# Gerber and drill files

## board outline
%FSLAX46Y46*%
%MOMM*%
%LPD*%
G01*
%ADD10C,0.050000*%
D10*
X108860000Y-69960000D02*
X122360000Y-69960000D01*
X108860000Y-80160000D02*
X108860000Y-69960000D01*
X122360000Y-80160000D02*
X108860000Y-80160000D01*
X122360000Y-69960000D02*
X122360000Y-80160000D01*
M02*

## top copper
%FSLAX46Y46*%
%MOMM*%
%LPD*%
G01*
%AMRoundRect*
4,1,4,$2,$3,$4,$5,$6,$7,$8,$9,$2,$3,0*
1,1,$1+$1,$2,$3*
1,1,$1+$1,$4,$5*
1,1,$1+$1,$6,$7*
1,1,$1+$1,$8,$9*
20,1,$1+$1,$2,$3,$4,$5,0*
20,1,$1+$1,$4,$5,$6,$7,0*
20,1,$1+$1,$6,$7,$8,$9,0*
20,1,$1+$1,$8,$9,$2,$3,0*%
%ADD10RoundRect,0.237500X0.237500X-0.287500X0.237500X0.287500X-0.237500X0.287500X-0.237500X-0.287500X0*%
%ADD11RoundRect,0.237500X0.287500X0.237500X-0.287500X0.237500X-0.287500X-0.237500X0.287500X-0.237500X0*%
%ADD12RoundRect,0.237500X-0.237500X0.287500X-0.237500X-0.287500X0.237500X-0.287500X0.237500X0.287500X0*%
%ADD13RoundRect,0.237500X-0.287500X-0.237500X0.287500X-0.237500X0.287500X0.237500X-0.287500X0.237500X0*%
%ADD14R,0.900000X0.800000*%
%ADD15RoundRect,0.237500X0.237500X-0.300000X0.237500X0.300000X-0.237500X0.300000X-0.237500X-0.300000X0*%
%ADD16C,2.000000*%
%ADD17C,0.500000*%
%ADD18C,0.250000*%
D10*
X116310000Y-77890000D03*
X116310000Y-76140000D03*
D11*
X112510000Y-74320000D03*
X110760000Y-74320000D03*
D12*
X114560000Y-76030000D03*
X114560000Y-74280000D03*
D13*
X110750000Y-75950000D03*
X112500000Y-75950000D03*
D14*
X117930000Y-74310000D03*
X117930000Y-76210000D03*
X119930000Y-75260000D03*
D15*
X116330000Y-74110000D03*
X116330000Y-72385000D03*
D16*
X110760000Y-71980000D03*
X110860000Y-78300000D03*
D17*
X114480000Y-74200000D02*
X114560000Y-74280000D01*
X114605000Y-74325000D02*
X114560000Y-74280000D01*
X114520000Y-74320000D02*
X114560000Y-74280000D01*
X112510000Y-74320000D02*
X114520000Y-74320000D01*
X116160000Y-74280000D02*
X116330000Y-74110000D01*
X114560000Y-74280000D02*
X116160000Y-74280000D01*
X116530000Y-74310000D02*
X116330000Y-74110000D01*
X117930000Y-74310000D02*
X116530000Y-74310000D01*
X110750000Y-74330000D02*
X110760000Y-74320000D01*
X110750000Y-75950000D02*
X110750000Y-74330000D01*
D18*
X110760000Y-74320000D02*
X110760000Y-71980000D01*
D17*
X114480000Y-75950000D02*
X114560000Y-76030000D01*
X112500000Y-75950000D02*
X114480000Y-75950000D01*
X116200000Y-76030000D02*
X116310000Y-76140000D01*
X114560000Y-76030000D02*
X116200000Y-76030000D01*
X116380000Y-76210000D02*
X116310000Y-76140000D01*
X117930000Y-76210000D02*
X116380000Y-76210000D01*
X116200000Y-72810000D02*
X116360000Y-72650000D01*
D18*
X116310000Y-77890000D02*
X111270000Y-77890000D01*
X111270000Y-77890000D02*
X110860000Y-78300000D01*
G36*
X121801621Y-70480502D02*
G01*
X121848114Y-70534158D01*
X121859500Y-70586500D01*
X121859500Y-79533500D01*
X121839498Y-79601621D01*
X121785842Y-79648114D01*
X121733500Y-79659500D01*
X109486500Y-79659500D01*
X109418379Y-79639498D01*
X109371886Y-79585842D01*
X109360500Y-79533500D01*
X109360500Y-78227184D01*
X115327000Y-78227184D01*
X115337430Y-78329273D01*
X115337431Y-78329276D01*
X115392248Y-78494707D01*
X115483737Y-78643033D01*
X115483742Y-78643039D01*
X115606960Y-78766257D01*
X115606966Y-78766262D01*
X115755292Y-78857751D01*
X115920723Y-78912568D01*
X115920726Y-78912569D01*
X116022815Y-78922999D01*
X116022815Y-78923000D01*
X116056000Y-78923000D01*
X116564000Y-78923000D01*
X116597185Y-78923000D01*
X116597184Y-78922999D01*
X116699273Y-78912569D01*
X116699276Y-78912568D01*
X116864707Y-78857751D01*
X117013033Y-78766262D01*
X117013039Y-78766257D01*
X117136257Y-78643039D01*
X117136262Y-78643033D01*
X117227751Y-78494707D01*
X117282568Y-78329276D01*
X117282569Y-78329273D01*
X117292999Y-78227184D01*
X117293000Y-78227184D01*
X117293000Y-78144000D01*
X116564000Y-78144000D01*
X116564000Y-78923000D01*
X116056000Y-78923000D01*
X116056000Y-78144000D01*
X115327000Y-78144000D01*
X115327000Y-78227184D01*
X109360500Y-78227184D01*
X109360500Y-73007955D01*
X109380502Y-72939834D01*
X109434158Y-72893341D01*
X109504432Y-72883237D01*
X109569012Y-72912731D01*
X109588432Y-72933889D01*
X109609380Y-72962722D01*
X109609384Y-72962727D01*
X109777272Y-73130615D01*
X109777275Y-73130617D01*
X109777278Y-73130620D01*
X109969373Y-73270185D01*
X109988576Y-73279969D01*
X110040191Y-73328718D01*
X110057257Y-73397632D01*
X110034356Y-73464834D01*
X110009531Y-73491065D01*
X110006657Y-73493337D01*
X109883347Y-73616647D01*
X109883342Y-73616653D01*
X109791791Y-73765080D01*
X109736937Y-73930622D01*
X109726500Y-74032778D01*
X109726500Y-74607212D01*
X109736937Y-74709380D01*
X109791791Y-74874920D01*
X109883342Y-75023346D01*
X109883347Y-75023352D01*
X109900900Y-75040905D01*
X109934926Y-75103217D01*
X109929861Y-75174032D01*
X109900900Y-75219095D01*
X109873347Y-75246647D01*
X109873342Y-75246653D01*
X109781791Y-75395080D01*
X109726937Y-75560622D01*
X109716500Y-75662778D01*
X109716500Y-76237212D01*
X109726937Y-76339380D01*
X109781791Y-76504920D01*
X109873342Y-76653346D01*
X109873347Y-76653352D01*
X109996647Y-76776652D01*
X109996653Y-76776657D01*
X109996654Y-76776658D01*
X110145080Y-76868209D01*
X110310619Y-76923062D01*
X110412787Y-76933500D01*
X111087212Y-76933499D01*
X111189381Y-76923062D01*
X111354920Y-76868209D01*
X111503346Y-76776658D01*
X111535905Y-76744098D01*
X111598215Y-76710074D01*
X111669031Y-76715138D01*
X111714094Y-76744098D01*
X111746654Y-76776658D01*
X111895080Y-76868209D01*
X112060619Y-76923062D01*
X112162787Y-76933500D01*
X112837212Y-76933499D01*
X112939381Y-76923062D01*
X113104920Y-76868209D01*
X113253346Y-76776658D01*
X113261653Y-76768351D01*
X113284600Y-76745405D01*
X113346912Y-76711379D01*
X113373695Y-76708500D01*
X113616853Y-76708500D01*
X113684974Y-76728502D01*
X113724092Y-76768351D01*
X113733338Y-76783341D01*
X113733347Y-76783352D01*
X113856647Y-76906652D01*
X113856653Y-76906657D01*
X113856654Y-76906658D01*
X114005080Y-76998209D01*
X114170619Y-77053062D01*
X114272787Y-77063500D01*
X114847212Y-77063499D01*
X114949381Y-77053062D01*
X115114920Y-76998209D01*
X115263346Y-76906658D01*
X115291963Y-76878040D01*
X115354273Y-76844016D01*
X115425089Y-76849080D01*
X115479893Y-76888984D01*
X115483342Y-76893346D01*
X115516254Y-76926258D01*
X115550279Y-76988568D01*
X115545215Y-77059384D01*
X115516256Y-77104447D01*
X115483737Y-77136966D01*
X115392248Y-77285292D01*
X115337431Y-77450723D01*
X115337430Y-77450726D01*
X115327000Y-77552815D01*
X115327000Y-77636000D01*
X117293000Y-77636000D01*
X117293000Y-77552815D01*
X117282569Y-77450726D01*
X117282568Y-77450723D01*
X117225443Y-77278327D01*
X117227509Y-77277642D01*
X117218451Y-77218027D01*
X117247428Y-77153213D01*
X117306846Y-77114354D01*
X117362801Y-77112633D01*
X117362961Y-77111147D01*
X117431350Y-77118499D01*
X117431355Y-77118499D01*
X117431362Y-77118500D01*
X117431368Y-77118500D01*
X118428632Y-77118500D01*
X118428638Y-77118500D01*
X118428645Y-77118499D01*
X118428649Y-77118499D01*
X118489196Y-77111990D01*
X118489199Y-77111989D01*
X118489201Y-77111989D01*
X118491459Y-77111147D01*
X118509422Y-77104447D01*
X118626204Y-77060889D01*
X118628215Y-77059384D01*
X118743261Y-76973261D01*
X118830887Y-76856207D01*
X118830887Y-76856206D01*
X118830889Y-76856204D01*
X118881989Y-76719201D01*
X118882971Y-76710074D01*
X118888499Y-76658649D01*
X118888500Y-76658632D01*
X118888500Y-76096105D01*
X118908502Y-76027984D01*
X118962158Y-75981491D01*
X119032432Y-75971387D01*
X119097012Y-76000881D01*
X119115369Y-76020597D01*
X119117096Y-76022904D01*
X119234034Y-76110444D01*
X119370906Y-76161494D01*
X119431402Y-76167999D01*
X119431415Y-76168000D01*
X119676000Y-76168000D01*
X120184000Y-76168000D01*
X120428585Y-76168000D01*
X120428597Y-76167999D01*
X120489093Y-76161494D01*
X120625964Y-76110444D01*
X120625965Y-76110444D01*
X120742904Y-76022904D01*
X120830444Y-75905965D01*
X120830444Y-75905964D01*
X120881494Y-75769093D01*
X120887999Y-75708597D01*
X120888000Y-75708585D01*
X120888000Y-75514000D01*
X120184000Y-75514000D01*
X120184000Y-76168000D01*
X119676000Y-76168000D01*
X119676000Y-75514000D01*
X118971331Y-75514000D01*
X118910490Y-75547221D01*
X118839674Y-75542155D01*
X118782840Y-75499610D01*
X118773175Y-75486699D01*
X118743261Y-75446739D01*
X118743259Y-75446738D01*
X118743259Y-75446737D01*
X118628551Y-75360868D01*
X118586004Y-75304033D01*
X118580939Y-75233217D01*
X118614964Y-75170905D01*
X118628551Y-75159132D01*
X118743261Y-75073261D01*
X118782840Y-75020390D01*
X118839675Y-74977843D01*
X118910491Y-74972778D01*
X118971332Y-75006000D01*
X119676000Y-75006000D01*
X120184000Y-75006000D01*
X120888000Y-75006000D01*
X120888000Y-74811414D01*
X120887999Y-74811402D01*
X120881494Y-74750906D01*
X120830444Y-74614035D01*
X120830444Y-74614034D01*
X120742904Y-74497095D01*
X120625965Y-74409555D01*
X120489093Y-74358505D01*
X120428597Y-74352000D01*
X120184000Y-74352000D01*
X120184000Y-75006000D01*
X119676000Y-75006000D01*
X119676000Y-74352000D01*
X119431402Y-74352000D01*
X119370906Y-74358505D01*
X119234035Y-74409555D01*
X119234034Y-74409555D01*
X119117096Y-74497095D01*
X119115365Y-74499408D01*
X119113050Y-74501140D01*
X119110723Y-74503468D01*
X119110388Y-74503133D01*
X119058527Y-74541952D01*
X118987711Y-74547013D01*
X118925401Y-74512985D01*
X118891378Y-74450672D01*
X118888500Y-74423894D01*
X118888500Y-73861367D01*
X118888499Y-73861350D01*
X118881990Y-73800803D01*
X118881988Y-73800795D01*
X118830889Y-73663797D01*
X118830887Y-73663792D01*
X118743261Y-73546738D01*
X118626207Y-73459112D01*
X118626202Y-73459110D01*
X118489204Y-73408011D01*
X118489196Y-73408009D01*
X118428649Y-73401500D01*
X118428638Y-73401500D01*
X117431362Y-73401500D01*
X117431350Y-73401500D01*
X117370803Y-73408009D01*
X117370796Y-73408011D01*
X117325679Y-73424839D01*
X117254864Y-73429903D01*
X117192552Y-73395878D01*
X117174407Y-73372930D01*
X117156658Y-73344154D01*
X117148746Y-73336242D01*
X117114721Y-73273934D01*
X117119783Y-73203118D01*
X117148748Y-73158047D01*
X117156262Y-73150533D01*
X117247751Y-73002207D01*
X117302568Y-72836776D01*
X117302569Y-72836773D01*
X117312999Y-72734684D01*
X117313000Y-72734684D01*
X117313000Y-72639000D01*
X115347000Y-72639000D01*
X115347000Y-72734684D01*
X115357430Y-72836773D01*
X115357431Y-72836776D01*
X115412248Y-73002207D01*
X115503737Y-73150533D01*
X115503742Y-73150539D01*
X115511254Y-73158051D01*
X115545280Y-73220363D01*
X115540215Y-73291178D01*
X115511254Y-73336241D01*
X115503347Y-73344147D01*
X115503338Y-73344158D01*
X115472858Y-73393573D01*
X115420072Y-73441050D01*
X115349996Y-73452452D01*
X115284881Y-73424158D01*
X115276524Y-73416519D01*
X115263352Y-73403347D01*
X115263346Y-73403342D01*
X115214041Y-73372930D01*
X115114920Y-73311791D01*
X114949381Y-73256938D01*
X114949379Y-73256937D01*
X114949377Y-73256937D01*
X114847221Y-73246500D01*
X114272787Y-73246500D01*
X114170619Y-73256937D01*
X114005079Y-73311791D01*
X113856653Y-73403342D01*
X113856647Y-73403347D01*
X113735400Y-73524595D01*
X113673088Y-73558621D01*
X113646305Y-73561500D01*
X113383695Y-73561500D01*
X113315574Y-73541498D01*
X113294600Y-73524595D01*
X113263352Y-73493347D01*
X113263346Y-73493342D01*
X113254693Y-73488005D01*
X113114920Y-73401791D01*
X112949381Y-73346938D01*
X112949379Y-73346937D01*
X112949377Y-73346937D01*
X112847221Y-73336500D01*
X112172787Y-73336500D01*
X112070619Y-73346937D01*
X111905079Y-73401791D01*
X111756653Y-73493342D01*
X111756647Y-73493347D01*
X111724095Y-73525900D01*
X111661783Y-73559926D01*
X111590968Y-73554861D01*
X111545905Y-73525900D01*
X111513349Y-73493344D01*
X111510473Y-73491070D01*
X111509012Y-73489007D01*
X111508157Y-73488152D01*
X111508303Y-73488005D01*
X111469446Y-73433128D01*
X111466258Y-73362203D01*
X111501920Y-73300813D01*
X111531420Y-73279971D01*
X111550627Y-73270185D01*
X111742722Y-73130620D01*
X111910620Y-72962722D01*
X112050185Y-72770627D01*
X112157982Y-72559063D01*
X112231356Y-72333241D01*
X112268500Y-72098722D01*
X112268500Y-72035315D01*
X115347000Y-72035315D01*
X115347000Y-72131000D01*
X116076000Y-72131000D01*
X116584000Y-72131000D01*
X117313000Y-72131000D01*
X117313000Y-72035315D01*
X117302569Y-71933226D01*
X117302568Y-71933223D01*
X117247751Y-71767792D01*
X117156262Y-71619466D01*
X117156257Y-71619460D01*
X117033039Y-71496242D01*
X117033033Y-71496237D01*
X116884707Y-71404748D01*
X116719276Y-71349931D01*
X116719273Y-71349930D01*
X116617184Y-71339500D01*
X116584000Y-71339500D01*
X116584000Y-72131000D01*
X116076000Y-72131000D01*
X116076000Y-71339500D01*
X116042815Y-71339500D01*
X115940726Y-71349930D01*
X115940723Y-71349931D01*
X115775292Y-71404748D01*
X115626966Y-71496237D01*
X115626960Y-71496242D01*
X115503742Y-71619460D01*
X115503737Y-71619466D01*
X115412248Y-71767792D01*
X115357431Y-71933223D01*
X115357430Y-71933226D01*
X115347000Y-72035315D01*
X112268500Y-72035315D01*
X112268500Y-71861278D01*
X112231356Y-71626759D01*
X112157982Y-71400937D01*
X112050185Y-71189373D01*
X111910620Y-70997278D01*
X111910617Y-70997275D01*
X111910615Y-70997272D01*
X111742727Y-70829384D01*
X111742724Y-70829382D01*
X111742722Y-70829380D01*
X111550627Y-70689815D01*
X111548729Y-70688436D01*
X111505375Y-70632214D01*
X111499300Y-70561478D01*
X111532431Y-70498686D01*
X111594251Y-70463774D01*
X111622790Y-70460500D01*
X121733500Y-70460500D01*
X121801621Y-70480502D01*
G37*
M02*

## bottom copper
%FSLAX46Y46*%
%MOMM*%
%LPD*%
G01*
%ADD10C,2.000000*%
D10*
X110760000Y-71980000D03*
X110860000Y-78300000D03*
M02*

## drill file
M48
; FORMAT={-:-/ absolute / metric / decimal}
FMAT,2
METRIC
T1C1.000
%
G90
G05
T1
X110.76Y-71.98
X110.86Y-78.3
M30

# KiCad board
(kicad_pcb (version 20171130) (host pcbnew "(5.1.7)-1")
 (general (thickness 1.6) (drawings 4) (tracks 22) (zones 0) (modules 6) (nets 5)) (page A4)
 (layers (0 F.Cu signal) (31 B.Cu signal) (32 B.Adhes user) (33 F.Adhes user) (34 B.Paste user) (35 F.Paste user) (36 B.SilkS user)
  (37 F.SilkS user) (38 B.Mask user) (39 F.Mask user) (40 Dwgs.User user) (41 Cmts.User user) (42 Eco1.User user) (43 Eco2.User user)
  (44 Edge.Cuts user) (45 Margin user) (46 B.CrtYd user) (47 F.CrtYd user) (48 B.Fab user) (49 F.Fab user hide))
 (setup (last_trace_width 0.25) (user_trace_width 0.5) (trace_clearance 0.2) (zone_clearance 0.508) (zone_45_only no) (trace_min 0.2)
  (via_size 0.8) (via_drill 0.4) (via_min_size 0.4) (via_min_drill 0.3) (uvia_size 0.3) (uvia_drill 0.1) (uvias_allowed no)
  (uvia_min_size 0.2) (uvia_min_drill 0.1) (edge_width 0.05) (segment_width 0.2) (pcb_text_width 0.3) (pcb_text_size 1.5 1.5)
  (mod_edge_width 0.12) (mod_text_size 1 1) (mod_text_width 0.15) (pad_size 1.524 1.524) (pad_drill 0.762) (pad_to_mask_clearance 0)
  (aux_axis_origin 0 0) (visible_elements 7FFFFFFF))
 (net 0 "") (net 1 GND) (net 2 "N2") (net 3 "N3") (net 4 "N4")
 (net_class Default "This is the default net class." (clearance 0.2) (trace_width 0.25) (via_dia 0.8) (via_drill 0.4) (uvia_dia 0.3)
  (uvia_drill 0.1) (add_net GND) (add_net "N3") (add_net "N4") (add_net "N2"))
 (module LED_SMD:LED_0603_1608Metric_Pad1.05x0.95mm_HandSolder (layer F.Cu) (at 116.31 77.015 90)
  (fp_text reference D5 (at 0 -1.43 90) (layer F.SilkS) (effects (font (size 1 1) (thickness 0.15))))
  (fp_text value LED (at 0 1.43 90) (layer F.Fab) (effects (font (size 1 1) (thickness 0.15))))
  (pad 1 smd roundrect (at -0.875 0 90) (size 1.05 0.95) (layers F.Cu F.Paste F.Mask) (roundrect_rratio 0.25) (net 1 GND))
  (pad 2 smd roundrect (at 0.875 0 90) (size 1.05 0.95) (layers F.Cu F.Paste F.Mask) (roundrect_rratio 0.25) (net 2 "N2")))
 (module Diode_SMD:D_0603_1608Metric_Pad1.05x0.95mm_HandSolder (layer F.Cu) (at 111.635 74.32 180)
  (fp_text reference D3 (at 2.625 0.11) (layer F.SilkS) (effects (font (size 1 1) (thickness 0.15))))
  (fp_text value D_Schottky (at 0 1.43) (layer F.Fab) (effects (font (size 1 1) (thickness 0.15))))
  (pad 1 smd roundrect (at -0.875 0 180) (size 1.05 0.95) (layers F.Cu F.Paste F.Mask) (roundrect_rratio 0.25) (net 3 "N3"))
  (pad 2 smd roundrect (at 0.875 0 180) (size 1.05 0.95) (layers F.Cu F.Paste F.Mask) (roundrect_rratio 0.25) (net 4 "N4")))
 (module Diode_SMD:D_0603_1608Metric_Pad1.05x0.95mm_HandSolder (layer F.Cu) (at 114.56 75.155 270)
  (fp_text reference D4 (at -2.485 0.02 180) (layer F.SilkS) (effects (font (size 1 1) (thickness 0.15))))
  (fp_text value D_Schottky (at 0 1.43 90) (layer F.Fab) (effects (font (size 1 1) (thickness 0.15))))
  (pad 2 smd roundrect (at 0.875 0 270) (size 1.05 0.95) (layers F.Cu F.Paste F.Mask) (roundrect_rratio 0.25) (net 2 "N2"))
  (pad 1 smd roundrect (at -0.875 0 270) (size 1.05 0.95) (layers F.Cu F.Paste F.Mask) (roundrect_rratio 0.25) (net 3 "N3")))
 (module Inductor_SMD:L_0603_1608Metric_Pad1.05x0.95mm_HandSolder (layer F.Cu) (at 111.625 75.95)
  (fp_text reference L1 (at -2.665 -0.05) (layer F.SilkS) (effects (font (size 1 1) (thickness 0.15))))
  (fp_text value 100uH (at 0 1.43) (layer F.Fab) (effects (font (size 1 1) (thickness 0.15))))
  (pad 1 smd roundrect (at -0.875 0) (size 1.05 0.95) (layers F.Cu F.Paste F.Mask) (roundrect_rratio 0.25) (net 4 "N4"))
  (pad 2 smd roundrect (at 0.875 0) (size 1.05 0.95) (layers F.Cu F.Paste F.Mask) (roundrect_rratio 0.25) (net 2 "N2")))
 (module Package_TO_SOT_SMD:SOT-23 (layer F.Cu) (at 118.93 75.26)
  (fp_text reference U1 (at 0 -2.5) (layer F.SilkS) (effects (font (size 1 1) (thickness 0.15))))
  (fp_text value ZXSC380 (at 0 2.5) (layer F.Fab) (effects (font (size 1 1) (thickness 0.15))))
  (pad 1 smd rect (at -1 -0.95) (size 0.9 0.8) (layers F.Cu F.Paste F.Mask) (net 3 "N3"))
  (pad 2 smd rect (at -1 0.95) (size 0.9 0.8) (layers F.Cu F.Paste F.Mask) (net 2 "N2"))
  (pad 3 smd rect (at 1 0) (size 0.9 0.8) (layers F.Cu F.Paste F.Mask) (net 1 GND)))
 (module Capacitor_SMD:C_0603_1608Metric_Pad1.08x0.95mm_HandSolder (layer F.Cu) (at 116.33 73.2475 90)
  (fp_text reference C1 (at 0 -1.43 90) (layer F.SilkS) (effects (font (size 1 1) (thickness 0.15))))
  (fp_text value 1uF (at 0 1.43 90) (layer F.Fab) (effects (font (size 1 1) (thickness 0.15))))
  (pad 1 smd roundrect (at -0.8625 0 90) (size 1.075 0.95) (layers F.Cu F.Paste F.Mask) (roundrect_rratio 0.25) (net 3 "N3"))
  (pad 2 smd roundrect (at 0.8625 0 90) (size 1.075 0.95) (layers F.Cu F.Paste F.Mask) (roundrect_rratio 0.25) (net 1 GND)))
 (gr_line (start 108.86 69.96) (end 122.36 69.96) (layer Edge.Cuts) (width 0.05))
 (gr_line (start 108.86 80.16) (end 108.86 69.96) (layer Edge.Cuts) (width 0.05))
 (gr_line (start 122.36 80.16) (end 108.86 80.16) (layer Edge.Cuts) (width 0.05))
 (gr_line (start 122.36 69.96) (end 122.36 80.16) (layer Edge.Cuts) (width 0.05))
 (segment (start 114.48 74.2) (end 114.56 74.28) (width 0.5) (layer F.Cu) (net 3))
 (segment (start 114.605 74.325) (end 114.56 74.28) (width 0.5) (layer F.Cu) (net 3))
 (segment (start 114.52 74.32) (end 114.56 74.28) (width 0.5) (layer F.Cu) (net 3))
 (segment (start 112.51 74.32) (end 114.52 74.32) (width 0.5) (layer F.Cu) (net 3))
 (segment (start 116.16 74.28) (end 116.33 74.11) (width 0.5) (layer F.Cu) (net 3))
 (segment (start 114.56 74.28) (end 116.16 74.28) (width 0.5) (layer F.Cu) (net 3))
 (segment (start 116.53 74.31) (end 116.33 74.11) (width 0.5) (layer F.Cu) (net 3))
 (segment (start 117.93 74.31) (end 116.53 74.31) (width 0.5) (layer F.Cu) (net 3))
 (segment (start 110.75 74.33) (end 110.76 74.32) (width 0.5) (layer F.Cu) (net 4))
 (segment (start 110.75 75.95) (end 110.75 74.33) (width 0.5) (layer F.Cu) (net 4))
 (segment (start 110.76 74.32) (end 110.76 71.98) (width 0.25) (layer F.Cu) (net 4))
 (via (at 110.76 71.98) (size 2) (drill 1) (layers F.Cu B.Cu) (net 4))
 (segment (start 114.48 75.95) (end 114.56 76.03) (width 0.5) (layer F.Cu) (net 2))
 (segment (start 112.5 75.95) (end 114.48 75.95) (width 0.5) (layer F.Cu) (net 2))
 (segment (start 116.2 76.03) (end 116.31 76.14) (width 0.5) (layer F.Cu) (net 2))
 (segment (start 114.56 76.03) (end 116.2 76.03) (width 0.5) (layer F.Cu) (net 2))
 (segment (start 116.38 76.21) (end 116.31 76.14) (width 0.5) (layer F.Cu) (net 2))
 (segment (start 117.93 76.21) (end 116.38 76.21) (width 0.5) (layer F.Cu) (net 2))
 (segment (start 116.2 72.81) (end 116.36 72.65) (width 0.5) (layer F.Cu) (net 1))
 (segment (start 116.31 77.89) (end 111.27 77.89) (width 0.25) (layer F.Cu) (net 1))
 (via (at 110.86 78.3) (size 2) (drill 1) (layers F.Cu B.Cu) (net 1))
 (segment (start 111.27 77.89) (end 110.86 78.3) (width 0.25) (layer F.Cu) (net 1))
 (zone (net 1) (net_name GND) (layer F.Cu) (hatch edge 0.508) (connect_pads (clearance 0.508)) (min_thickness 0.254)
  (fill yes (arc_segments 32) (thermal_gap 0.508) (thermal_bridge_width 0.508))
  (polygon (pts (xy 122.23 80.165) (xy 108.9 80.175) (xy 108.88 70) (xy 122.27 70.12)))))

